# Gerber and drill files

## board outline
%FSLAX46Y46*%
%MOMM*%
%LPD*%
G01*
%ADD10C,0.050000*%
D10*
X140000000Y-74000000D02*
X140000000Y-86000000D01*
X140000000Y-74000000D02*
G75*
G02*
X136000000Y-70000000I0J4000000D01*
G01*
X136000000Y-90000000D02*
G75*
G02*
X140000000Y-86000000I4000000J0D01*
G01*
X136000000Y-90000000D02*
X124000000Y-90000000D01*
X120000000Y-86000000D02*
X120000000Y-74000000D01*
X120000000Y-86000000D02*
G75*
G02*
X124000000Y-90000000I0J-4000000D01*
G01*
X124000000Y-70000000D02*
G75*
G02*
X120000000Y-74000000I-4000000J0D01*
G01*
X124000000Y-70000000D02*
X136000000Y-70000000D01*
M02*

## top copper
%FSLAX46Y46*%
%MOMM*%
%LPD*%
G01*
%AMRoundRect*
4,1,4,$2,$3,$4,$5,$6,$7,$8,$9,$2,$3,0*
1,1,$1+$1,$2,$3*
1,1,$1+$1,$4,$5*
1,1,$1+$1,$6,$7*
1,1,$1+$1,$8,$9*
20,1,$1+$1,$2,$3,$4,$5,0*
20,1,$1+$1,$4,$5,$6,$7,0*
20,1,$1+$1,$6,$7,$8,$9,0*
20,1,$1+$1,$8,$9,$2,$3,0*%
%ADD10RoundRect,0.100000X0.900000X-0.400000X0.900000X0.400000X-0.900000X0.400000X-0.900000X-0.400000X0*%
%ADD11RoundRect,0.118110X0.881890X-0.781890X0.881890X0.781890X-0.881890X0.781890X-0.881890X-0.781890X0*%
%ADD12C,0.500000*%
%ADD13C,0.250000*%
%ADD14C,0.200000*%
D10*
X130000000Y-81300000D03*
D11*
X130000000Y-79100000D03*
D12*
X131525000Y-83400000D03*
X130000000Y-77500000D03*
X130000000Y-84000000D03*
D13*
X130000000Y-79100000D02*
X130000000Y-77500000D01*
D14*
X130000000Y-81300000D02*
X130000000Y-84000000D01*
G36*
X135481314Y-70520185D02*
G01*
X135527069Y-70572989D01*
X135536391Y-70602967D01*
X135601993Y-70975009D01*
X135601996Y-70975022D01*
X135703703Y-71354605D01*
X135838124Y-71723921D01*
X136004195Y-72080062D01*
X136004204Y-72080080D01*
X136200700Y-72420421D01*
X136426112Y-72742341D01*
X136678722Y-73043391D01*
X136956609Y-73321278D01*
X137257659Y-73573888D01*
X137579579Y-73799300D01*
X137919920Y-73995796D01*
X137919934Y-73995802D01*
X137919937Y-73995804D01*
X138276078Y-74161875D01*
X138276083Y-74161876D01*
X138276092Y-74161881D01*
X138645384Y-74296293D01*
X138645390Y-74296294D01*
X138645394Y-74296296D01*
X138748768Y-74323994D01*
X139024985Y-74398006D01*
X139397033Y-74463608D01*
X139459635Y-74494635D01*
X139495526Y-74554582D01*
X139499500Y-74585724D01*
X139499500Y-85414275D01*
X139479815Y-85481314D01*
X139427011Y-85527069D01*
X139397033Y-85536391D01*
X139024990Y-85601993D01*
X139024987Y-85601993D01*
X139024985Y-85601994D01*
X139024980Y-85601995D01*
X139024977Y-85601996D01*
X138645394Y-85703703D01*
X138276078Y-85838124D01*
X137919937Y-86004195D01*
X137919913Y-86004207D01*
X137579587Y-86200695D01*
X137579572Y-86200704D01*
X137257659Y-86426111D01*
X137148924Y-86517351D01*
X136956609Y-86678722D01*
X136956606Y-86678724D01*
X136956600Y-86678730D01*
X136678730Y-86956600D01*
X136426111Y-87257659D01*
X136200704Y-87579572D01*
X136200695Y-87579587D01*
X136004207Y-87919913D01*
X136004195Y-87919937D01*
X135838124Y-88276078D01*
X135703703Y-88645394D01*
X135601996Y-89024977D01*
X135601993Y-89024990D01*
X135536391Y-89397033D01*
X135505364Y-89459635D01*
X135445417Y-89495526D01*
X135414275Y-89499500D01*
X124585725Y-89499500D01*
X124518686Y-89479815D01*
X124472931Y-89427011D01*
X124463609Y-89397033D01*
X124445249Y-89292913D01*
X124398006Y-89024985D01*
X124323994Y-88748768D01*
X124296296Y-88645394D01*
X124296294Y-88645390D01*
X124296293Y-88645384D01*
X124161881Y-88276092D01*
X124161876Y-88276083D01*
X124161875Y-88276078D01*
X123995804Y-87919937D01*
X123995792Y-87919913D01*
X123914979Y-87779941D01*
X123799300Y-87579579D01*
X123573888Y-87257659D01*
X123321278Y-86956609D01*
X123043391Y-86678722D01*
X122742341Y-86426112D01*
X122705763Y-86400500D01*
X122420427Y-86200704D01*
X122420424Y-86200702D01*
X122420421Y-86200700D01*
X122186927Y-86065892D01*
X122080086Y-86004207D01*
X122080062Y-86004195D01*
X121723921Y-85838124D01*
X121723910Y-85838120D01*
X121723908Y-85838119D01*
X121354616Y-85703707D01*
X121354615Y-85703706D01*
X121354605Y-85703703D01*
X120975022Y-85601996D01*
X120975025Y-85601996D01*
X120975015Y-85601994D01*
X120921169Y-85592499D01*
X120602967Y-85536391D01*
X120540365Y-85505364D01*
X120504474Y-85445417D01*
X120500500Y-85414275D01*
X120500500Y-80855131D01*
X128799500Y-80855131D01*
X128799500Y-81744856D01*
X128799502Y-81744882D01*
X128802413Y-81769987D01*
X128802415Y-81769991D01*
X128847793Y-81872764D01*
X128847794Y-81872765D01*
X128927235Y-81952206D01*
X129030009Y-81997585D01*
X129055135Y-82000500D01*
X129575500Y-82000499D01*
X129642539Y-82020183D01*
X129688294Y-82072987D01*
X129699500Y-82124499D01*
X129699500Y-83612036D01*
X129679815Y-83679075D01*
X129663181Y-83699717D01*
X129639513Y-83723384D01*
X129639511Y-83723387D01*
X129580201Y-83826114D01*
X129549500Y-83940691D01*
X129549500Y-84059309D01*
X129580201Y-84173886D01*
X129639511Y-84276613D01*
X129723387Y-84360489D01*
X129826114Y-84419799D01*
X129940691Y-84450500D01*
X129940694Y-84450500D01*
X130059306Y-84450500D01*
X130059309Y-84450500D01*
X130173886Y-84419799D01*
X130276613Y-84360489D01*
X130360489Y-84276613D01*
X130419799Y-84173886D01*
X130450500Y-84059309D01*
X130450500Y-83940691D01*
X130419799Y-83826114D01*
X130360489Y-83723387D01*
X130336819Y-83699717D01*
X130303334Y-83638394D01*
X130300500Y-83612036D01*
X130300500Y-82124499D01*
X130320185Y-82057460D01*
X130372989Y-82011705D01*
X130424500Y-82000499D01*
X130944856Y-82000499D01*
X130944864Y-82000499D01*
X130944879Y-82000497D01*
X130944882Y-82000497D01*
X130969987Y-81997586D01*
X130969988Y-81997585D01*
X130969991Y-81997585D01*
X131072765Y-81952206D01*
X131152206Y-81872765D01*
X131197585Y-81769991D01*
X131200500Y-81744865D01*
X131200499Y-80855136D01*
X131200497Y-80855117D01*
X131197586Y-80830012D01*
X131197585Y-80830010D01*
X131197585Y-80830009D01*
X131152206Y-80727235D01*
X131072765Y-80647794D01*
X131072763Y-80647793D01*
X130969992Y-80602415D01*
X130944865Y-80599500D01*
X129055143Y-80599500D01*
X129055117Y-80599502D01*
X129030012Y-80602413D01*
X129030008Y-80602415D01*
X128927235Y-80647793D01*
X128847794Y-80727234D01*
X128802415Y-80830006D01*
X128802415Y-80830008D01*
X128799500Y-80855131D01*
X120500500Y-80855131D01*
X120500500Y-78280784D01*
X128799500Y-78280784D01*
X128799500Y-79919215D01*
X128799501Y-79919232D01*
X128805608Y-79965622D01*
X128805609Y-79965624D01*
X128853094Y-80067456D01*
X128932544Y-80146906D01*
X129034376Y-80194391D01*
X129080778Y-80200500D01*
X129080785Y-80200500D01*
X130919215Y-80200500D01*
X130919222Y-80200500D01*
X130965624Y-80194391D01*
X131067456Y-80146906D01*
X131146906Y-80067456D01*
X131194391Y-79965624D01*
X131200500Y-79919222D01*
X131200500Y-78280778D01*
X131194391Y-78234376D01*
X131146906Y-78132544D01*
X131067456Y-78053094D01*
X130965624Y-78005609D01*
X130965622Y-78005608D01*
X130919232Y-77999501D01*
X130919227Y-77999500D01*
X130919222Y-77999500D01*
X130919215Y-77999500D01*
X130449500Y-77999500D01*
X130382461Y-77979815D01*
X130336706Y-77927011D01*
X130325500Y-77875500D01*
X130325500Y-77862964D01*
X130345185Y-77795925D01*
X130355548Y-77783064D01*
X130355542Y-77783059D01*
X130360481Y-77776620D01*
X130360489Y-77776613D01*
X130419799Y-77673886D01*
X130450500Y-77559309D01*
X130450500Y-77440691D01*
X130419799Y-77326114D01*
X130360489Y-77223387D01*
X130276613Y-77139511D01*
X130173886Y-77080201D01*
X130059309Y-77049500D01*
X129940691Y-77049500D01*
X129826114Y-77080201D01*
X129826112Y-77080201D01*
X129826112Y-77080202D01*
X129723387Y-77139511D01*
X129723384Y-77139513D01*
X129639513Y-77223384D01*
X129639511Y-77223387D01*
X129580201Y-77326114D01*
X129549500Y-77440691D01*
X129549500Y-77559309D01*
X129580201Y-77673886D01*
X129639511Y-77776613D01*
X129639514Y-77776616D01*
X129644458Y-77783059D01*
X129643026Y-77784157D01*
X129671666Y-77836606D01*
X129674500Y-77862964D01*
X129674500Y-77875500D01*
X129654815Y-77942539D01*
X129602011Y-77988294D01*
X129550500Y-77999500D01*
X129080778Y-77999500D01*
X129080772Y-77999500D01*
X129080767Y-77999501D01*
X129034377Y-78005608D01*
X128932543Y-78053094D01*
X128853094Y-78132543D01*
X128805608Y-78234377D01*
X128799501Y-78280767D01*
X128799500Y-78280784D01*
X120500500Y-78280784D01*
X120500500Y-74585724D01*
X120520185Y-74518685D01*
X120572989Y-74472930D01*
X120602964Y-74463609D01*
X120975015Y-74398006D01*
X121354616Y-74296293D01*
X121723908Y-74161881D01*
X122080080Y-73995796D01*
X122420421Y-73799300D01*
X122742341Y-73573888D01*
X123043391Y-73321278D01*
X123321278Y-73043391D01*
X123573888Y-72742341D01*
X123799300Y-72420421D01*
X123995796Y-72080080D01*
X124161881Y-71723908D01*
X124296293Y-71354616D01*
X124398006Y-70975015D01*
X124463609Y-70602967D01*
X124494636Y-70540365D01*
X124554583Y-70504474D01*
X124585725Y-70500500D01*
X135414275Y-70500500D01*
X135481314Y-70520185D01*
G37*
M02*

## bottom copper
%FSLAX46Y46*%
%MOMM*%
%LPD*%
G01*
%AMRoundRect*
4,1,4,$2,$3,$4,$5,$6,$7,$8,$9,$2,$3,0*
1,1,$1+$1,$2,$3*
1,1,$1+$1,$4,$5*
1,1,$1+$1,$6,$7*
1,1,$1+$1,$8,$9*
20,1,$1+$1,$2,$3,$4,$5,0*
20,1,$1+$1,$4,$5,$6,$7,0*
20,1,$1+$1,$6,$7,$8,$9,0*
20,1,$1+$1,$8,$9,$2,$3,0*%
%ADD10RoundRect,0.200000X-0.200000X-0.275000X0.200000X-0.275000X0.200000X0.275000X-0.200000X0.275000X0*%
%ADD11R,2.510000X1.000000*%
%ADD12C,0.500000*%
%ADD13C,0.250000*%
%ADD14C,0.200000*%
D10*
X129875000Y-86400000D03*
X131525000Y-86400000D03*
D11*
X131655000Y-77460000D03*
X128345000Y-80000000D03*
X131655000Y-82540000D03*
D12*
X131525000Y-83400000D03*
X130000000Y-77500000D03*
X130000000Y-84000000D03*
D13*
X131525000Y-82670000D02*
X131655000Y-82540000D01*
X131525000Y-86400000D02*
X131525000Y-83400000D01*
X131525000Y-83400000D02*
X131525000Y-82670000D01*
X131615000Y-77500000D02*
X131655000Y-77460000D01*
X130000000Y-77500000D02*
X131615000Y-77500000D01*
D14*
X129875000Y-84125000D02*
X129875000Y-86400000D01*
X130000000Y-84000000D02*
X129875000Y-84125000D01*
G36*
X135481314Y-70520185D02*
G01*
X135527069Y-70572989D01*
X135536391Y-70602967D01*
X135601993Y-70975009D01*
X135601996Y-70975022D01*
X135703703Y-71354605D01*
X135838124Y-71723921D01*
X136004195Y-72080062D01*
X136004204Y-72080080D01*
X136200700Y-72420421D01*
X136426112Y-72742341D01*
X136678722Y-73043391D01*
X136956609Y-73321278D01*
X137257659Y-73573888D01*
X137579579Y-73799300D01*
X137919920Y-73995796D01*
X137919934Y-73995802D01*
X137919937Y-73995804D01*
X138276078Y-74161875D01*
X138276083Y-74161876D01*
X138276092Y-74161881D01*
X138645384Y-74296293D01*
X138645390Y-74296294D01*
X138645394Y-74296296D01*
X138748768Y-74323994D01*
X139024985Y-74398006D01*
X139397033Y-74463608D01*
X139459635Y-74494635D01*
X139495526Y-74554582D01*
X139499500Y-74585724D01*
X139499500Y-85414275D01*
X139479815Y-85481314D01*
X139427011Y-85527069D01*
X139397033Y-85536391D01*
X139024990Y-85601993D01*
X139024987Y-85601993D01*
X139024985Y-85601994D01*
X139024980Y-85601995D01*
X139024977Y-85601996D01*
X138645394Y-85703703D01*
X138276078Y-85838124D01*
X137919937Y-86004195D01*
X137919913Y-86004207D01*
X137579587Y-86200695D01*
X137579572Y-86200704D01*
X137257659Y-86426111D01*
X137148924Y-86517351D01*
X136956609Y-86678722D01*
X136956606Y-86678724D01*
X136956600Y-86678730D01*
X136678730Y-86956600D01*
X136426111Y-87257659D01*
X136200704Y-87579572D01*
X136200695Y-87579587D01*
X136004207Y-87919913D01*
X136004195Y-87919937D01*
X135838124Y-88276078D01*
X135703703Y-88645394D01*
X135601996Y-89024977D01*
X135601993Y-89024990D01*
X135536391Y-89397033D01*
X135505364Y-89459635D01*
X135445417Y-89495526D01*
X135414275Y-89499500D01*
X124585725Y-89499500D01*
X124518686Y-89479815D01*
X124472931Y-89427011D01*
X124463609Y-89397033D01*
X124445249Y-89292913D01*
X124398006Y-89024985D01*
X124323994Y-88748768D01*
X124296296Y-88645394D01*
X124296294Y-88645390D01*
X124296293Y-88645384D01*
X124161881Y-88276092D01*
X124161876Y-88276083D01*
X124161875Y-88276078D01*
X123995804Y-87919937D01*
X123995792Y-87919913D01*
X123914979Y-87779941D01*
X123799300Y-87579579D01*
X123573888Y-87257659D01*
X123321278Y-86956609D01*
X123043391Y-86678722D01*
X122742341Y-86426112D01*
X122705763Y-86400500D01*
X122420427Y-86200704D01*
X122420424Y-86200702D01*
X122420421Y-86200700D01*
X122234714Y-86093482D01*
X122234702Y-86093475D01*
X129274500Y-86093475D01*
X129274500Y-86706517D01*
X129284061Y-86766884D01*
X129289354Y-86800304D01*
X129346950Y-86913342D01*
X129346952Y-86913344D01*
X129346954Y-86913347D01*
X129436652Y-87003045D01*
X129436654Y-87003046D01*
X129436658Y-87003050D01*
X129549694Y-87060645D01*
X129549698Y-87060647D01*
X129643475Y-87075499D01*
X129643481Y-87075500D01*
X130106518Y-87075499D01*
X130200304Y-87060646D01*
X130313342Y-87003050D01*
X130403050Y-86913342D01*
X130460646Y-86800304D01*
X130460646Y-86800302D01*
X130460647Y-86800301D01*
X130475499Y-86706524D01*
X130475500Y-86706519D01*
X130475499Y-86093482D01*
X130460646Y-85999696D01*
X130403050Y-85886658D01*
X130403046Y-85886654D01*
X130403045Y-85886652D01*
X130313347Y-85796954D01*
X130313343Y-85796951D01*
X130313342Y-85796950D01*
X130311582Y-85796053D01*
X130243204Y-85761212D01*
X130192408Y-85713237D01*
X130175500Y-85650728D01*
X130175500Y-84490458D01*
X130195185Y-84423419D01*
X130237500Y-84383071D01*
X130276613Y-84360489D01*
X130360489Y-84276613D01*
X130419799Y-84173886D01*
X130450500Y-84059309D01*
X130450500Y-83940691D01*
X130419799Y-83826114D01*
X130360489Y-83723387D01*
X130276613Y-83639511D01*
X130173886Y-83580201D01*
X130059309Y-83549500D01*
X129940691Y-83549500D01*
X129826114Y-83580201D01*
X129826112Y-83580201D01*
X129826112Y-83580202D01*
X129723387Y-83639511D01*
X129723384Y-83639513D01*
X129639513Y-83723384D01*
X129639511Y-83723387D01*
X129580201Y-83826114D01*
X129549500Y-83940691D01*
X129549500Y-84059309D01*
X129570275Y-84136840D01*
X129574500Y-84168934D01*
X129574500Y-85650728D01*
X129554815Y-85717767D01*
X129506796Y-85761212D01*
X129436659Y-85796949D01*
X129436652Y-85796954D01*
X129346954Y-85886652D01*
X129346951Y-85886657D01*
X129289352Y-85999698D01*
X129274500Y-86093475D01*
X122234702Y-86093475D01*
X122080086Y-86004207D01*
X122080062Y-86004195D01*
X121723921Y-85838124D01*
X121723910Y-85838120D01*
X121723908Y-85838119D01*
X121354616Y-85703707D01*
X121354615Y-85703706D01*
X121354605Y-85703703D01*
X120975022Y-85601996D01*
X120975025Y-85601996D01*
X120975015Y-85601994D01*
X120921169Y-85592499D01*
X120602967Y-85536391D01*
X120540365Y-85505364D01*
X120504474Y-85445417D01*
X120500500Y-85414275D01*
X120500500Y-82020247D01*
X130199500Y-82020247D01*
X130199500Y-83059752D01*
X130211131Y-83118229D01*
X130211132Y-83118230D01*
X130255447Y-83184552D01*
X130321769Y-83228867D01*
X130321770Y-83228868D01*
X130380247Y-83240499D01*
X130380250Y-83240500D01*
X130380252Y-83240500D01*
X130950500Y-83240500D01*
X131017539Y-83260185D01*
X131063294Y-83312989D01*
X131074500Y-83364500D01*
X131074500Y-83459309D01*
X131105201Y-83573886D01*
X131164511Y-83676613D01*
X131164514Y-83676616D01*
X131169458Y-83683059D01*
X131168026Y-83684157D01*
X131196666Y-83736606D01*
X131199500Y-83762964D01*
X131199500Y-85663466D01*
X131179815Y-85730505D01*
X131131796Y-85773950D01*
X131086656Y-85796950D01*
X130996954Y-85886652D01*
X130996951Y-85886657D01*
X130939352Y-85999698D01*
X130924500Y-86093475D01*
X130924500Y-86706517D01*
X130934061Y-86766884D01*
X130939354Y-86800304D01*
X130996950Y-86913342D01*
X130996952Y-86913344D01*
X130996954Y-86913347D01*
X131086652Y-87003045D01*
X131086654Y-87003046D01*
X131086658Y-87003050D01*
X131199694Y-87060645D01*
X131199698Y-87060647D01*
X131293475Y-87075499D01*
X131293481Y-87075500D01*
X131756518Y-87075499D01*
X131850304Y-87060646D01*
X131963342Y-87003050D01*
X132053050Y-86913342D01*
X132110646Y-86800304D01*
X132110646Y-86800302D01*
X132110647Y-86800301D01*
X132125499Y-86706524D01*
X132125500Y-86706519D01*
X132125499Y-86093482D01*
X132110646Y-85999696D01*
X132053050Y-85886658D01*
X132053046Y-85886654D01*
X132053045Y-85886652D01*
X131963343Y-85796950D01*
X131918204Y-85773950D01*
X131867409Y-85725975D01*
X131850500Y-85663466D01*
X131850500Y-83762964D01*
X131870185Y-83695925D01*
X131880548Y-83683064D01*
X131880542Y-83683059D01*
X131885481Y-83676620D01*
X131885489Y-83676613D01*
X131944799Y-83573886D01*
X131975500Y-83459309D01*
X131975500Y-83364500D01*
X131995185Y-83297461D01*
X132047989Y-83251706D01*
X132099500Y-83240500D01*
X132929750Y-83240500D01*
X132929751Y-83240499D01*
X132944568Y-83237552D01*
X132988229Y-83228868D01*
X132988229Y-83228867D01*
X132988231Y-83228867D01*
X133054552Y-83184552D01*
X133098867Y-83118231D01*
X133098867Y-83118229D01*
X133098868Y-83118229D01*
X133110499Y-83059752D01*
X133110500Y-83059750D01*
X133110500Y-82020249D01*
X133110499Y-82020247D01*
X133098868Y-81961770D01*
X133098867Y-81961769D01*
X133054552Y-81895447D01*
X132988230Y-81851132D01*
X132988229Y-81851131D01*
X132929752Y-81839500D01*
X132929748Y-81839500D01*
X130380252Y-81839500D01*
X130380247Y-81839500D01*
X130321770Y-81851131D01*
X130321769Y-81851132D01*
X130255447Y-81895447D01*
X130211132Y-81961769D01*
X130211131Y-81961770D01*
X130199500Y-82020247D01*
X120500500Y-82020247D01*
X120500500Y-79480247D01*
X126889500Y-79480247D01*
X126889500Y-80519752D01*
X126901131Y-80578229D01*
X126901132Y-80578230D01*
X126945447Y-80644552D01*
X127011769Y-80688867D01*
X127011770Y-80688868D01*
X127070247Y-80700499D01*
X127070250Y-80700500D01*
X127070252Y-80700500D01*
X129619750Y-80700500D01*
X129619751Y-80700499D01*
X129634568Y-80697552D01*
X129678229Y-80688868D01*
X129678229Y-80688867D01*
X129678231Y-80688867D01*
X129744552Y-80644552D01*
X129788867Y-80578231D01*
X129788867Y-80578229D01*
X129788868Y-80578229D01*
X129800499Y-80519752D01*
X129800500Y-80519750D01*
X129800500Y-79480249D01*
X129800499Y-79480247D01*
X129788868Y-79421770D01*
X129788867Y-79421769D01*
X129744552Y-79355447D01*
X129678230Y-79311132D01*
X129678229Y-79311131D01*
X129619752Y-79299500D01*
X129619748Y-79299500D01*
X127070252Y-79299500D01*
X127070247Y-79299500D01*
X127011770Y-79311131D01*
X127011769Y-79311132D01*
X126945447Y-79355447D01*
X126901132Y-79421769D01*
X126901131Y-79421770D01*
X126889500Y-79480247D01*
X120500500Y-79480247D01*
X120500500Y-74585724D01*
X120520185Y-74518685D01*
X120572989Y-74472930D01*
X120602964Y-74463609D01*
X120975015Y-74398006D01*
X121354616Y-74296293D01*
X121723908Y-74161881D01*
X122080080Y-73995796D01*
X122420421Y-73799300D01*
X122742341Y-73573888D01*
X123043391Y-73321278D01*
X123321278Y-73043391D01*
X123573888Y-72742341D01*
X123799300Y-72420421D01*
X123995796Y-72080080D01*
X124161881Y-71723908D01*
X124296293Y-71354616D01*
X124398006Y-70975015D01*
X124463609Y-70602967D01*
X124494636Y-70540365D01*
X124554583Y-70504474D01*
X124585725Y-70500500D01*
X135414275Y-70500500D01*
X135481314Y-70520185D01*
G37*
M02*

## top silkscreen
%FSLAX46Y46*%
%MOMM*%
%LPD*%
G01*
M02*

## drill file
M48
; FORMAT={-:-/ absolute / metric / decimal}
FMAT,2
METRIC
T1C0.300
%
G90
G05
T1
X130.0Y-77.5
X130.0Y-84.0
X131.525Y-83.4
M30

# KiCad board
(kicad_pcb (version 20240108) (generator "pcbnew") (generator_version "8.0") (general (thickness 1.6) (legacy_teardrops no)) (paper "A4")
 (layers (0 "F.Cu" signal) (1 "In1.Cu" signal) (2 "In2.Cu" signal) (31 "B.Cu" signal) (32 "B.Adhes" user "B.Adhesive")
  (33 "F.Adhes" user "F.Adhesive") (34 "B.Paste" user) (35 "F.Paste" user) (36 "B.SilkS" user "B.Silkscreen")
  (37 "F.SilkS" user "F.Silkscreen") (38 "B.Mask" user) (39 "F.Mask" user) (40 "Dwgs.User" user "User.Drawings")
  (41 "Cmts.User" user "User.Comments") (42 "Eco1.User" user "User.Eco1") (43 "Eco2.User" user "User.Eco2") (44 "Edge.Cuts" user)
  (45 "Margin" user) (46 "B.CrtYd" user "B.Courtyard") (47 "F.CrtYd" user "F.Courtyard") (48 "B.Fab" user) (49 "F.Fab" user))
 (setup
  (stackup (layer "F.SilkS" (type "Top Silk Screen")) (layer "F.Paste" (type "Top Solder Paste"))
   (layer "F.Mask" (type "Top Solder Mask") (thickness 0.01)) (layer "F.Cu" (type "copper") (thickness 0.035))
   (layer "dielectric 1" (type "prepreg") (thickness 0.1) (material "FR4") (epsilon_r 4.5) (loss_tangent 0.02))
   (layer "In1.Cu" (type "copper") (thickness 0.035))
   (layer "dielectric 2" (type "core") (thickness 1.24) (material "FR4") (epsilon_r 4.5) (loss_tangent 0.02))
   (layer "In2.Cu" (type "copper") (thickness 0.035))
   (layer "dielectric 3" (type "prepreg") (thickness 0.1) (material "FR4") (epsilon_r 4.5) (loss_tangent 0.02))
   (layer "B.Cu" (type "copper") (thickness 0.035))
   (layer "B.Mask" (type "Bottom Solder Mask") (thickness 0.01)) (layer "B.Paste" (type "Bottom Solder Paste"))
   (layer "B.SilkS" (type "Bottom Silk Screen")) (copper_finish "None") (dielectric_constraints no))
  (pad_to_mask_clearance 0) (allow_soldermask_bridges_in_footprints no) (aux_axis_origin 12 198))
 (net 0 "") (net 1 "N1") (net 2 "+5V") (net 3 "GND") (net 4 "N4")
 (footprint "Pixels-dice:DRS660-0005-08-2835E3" (layer "F.Cu") (at 130 80 90)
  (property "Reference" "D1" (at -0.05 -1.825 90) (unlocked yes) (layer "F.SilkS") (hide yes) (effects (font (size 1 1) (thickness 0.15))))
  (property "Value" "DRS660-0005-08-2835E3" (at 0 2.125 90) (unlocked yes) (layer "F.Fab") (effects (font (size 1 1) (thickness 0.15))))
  (pad "1" smd roundrect (at -1.3 0 90) (size 1 2) (layers "F.Cu" "F.Paste" "F.Mask") (roundrect_rratio 0.1) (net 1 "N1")
   (thermal_bridge_angle 45))
  (pad "2" smd roundrect (at 0.9 0 90) (size 1.8 2) (layers "F.Cu" "F.Paste" "F.Mask") (roundrect_rratio 0.0656167979) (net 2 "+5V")
   (thermal_bridge_angle 45)))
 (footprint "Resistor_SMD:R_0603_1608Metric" (layer "B.Cu") (at 130.7 86.4)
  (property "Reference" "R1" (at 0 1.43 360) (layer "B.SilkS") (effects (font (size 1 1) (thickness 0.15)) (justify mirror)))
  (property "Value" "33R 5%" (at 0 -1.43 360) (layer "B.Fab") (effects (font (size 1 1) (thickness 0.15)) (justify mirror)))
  (pad "1" smd roundrect (at -0.825 0) (size 0.8 0.95) (layers "B.Cu" "B.Paste" "B.Mask") (roundrect_rratio 0.25) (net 1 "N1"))
  (pad "2" smd roundrect (at 0.825 0) (size 0.8 0.95) (layers "B.Cu" "B.Paste" "B.Mask") (roundrect_rratio 0.25) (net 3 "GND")))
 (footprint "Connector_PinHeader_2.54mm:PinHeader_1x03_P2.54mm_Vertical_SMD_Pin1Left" (layer "B.Cu") (at 130 80 180)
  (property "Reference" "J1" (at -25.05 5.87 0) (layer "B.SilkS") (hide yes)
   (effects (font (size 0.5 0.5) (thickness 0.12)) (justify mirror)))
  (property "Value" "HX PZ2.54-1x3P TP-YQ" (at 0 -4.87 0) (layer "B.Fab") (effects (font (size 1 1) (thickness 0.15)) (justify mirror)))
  (pad "1" smd rect (at -1.655 2.54 180) (size 2.51 1) (layers "B.Cu" "B.Paste" "B.Mask") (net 2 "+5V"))
  (pad "2" smd rect (at 1.655 0 180) (size 2.51 1) (layers "B.Cu" "B.Paste" "B.Mask") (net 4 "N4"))
  (pad "3" smd rect (at -1.655 -2.54 180) (size 2.51 1) (layers "B.Cu" "B.Paste" "B.Mask") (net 3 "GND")))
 (gr_line (start 140 74) (end 140 86) (stroke (width 0.05) (type default)) (layer "Edge.Cuts"))
 (gr_arc (start 140 74) (mid 137.171573 72.828427) (end 136 70) (stroke (width 0.05) (type default)) (layer "Edge.Cuts"))
 (gr_arc (start 136 90) (mid 137.171573 87.171573) (end 140 86) (stroke (width 0.05) (type default)) (layer "Edge.Cuts"))
 (gr_line (start 136 90) (end 124 90) (stroke (width 0.05) (type default)) (layer "Edge.Cuts"))
 (gr_line (start 120 86) (end 120 74) (stroke (width 0.05) (type default)) (layer "Edge.Cuts"))
 (gr_arc (start 120 86) (mid 122.828427 87.171573) (end 124 90) (stroke (width 0.05) (type default)) (layer "Edge.Cuts"))
 (gr_arc (start 124 70) (mid 122.828427 72.828427) (end 120 74) (stroke (width 0.05) (type default)) (layer "Edge.Cuts"))
 (gr_line (start 124 70) (end 136 70) (stroke (width 0.05) (type default)) (layer "Edge.Cuts"))
 (via (at 131.525 83.4) (size 0.5) (drill 0.3) (layers "F.Cu" "B.Cu") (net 3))
 (segment (start 131.525 82.67) (end 131.655 82.54) (width 0.25) (layer "B.Cu") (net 3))
 (segment (start 131.525 86.4) (end 131.525 83.4) (width 0.25) (layer "B.Cu") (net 3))
 (segment (start 131.525 83.4) (end 131.525 82.67) (width 0.25) (layer "B.Cu") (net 3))
 (segment (start 130 79.1) (end 130 77.5) (width 0.25) (layer "F.Cu") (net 2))
 (via (at 130 77.5) (size 0.5) (drill 0.3) (layers "F.Cu" "B.Cu") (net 2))
 (segment (start 131.615 77.5) (end 131.655 77.46) (width 0.25) (layer "B.Cu") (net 2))
 (segment (start 130 77.5) (end 131.615 77.5) (width 0.25) (layer "B.Cu") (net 2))
 (segment (start 130 81.3) (end 130 84) (width 0.2) (layer "F.Cu") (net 1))
 (via (at 130 84) (size 0.5) (drill 0.3) (layers "F.Cu" "B.Cu") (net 1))
 (segment (start 129.875 84.125) (end 129.875 86.4) (width 0.2) (layer "B.Cu") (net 1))
 (segment (start 130 84) (end 129.875 84.125) (width 0.2) (layer "B.Cu") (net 1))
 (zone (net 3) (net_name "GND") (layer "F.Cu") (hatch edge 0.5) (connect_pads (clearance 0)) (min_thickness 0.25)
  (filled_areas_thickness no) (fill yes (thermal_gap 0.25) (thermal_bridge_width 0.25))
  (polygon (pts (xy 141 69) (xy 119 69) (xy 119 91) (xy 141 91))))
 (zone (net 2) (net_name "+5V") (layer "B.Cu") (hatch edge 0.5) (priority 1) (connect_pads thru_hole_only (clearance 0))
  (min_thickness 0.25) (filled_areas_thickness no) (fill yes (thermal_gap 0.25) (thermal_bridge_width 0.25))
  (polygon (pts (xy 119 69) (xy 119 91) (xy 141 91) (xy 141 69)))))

